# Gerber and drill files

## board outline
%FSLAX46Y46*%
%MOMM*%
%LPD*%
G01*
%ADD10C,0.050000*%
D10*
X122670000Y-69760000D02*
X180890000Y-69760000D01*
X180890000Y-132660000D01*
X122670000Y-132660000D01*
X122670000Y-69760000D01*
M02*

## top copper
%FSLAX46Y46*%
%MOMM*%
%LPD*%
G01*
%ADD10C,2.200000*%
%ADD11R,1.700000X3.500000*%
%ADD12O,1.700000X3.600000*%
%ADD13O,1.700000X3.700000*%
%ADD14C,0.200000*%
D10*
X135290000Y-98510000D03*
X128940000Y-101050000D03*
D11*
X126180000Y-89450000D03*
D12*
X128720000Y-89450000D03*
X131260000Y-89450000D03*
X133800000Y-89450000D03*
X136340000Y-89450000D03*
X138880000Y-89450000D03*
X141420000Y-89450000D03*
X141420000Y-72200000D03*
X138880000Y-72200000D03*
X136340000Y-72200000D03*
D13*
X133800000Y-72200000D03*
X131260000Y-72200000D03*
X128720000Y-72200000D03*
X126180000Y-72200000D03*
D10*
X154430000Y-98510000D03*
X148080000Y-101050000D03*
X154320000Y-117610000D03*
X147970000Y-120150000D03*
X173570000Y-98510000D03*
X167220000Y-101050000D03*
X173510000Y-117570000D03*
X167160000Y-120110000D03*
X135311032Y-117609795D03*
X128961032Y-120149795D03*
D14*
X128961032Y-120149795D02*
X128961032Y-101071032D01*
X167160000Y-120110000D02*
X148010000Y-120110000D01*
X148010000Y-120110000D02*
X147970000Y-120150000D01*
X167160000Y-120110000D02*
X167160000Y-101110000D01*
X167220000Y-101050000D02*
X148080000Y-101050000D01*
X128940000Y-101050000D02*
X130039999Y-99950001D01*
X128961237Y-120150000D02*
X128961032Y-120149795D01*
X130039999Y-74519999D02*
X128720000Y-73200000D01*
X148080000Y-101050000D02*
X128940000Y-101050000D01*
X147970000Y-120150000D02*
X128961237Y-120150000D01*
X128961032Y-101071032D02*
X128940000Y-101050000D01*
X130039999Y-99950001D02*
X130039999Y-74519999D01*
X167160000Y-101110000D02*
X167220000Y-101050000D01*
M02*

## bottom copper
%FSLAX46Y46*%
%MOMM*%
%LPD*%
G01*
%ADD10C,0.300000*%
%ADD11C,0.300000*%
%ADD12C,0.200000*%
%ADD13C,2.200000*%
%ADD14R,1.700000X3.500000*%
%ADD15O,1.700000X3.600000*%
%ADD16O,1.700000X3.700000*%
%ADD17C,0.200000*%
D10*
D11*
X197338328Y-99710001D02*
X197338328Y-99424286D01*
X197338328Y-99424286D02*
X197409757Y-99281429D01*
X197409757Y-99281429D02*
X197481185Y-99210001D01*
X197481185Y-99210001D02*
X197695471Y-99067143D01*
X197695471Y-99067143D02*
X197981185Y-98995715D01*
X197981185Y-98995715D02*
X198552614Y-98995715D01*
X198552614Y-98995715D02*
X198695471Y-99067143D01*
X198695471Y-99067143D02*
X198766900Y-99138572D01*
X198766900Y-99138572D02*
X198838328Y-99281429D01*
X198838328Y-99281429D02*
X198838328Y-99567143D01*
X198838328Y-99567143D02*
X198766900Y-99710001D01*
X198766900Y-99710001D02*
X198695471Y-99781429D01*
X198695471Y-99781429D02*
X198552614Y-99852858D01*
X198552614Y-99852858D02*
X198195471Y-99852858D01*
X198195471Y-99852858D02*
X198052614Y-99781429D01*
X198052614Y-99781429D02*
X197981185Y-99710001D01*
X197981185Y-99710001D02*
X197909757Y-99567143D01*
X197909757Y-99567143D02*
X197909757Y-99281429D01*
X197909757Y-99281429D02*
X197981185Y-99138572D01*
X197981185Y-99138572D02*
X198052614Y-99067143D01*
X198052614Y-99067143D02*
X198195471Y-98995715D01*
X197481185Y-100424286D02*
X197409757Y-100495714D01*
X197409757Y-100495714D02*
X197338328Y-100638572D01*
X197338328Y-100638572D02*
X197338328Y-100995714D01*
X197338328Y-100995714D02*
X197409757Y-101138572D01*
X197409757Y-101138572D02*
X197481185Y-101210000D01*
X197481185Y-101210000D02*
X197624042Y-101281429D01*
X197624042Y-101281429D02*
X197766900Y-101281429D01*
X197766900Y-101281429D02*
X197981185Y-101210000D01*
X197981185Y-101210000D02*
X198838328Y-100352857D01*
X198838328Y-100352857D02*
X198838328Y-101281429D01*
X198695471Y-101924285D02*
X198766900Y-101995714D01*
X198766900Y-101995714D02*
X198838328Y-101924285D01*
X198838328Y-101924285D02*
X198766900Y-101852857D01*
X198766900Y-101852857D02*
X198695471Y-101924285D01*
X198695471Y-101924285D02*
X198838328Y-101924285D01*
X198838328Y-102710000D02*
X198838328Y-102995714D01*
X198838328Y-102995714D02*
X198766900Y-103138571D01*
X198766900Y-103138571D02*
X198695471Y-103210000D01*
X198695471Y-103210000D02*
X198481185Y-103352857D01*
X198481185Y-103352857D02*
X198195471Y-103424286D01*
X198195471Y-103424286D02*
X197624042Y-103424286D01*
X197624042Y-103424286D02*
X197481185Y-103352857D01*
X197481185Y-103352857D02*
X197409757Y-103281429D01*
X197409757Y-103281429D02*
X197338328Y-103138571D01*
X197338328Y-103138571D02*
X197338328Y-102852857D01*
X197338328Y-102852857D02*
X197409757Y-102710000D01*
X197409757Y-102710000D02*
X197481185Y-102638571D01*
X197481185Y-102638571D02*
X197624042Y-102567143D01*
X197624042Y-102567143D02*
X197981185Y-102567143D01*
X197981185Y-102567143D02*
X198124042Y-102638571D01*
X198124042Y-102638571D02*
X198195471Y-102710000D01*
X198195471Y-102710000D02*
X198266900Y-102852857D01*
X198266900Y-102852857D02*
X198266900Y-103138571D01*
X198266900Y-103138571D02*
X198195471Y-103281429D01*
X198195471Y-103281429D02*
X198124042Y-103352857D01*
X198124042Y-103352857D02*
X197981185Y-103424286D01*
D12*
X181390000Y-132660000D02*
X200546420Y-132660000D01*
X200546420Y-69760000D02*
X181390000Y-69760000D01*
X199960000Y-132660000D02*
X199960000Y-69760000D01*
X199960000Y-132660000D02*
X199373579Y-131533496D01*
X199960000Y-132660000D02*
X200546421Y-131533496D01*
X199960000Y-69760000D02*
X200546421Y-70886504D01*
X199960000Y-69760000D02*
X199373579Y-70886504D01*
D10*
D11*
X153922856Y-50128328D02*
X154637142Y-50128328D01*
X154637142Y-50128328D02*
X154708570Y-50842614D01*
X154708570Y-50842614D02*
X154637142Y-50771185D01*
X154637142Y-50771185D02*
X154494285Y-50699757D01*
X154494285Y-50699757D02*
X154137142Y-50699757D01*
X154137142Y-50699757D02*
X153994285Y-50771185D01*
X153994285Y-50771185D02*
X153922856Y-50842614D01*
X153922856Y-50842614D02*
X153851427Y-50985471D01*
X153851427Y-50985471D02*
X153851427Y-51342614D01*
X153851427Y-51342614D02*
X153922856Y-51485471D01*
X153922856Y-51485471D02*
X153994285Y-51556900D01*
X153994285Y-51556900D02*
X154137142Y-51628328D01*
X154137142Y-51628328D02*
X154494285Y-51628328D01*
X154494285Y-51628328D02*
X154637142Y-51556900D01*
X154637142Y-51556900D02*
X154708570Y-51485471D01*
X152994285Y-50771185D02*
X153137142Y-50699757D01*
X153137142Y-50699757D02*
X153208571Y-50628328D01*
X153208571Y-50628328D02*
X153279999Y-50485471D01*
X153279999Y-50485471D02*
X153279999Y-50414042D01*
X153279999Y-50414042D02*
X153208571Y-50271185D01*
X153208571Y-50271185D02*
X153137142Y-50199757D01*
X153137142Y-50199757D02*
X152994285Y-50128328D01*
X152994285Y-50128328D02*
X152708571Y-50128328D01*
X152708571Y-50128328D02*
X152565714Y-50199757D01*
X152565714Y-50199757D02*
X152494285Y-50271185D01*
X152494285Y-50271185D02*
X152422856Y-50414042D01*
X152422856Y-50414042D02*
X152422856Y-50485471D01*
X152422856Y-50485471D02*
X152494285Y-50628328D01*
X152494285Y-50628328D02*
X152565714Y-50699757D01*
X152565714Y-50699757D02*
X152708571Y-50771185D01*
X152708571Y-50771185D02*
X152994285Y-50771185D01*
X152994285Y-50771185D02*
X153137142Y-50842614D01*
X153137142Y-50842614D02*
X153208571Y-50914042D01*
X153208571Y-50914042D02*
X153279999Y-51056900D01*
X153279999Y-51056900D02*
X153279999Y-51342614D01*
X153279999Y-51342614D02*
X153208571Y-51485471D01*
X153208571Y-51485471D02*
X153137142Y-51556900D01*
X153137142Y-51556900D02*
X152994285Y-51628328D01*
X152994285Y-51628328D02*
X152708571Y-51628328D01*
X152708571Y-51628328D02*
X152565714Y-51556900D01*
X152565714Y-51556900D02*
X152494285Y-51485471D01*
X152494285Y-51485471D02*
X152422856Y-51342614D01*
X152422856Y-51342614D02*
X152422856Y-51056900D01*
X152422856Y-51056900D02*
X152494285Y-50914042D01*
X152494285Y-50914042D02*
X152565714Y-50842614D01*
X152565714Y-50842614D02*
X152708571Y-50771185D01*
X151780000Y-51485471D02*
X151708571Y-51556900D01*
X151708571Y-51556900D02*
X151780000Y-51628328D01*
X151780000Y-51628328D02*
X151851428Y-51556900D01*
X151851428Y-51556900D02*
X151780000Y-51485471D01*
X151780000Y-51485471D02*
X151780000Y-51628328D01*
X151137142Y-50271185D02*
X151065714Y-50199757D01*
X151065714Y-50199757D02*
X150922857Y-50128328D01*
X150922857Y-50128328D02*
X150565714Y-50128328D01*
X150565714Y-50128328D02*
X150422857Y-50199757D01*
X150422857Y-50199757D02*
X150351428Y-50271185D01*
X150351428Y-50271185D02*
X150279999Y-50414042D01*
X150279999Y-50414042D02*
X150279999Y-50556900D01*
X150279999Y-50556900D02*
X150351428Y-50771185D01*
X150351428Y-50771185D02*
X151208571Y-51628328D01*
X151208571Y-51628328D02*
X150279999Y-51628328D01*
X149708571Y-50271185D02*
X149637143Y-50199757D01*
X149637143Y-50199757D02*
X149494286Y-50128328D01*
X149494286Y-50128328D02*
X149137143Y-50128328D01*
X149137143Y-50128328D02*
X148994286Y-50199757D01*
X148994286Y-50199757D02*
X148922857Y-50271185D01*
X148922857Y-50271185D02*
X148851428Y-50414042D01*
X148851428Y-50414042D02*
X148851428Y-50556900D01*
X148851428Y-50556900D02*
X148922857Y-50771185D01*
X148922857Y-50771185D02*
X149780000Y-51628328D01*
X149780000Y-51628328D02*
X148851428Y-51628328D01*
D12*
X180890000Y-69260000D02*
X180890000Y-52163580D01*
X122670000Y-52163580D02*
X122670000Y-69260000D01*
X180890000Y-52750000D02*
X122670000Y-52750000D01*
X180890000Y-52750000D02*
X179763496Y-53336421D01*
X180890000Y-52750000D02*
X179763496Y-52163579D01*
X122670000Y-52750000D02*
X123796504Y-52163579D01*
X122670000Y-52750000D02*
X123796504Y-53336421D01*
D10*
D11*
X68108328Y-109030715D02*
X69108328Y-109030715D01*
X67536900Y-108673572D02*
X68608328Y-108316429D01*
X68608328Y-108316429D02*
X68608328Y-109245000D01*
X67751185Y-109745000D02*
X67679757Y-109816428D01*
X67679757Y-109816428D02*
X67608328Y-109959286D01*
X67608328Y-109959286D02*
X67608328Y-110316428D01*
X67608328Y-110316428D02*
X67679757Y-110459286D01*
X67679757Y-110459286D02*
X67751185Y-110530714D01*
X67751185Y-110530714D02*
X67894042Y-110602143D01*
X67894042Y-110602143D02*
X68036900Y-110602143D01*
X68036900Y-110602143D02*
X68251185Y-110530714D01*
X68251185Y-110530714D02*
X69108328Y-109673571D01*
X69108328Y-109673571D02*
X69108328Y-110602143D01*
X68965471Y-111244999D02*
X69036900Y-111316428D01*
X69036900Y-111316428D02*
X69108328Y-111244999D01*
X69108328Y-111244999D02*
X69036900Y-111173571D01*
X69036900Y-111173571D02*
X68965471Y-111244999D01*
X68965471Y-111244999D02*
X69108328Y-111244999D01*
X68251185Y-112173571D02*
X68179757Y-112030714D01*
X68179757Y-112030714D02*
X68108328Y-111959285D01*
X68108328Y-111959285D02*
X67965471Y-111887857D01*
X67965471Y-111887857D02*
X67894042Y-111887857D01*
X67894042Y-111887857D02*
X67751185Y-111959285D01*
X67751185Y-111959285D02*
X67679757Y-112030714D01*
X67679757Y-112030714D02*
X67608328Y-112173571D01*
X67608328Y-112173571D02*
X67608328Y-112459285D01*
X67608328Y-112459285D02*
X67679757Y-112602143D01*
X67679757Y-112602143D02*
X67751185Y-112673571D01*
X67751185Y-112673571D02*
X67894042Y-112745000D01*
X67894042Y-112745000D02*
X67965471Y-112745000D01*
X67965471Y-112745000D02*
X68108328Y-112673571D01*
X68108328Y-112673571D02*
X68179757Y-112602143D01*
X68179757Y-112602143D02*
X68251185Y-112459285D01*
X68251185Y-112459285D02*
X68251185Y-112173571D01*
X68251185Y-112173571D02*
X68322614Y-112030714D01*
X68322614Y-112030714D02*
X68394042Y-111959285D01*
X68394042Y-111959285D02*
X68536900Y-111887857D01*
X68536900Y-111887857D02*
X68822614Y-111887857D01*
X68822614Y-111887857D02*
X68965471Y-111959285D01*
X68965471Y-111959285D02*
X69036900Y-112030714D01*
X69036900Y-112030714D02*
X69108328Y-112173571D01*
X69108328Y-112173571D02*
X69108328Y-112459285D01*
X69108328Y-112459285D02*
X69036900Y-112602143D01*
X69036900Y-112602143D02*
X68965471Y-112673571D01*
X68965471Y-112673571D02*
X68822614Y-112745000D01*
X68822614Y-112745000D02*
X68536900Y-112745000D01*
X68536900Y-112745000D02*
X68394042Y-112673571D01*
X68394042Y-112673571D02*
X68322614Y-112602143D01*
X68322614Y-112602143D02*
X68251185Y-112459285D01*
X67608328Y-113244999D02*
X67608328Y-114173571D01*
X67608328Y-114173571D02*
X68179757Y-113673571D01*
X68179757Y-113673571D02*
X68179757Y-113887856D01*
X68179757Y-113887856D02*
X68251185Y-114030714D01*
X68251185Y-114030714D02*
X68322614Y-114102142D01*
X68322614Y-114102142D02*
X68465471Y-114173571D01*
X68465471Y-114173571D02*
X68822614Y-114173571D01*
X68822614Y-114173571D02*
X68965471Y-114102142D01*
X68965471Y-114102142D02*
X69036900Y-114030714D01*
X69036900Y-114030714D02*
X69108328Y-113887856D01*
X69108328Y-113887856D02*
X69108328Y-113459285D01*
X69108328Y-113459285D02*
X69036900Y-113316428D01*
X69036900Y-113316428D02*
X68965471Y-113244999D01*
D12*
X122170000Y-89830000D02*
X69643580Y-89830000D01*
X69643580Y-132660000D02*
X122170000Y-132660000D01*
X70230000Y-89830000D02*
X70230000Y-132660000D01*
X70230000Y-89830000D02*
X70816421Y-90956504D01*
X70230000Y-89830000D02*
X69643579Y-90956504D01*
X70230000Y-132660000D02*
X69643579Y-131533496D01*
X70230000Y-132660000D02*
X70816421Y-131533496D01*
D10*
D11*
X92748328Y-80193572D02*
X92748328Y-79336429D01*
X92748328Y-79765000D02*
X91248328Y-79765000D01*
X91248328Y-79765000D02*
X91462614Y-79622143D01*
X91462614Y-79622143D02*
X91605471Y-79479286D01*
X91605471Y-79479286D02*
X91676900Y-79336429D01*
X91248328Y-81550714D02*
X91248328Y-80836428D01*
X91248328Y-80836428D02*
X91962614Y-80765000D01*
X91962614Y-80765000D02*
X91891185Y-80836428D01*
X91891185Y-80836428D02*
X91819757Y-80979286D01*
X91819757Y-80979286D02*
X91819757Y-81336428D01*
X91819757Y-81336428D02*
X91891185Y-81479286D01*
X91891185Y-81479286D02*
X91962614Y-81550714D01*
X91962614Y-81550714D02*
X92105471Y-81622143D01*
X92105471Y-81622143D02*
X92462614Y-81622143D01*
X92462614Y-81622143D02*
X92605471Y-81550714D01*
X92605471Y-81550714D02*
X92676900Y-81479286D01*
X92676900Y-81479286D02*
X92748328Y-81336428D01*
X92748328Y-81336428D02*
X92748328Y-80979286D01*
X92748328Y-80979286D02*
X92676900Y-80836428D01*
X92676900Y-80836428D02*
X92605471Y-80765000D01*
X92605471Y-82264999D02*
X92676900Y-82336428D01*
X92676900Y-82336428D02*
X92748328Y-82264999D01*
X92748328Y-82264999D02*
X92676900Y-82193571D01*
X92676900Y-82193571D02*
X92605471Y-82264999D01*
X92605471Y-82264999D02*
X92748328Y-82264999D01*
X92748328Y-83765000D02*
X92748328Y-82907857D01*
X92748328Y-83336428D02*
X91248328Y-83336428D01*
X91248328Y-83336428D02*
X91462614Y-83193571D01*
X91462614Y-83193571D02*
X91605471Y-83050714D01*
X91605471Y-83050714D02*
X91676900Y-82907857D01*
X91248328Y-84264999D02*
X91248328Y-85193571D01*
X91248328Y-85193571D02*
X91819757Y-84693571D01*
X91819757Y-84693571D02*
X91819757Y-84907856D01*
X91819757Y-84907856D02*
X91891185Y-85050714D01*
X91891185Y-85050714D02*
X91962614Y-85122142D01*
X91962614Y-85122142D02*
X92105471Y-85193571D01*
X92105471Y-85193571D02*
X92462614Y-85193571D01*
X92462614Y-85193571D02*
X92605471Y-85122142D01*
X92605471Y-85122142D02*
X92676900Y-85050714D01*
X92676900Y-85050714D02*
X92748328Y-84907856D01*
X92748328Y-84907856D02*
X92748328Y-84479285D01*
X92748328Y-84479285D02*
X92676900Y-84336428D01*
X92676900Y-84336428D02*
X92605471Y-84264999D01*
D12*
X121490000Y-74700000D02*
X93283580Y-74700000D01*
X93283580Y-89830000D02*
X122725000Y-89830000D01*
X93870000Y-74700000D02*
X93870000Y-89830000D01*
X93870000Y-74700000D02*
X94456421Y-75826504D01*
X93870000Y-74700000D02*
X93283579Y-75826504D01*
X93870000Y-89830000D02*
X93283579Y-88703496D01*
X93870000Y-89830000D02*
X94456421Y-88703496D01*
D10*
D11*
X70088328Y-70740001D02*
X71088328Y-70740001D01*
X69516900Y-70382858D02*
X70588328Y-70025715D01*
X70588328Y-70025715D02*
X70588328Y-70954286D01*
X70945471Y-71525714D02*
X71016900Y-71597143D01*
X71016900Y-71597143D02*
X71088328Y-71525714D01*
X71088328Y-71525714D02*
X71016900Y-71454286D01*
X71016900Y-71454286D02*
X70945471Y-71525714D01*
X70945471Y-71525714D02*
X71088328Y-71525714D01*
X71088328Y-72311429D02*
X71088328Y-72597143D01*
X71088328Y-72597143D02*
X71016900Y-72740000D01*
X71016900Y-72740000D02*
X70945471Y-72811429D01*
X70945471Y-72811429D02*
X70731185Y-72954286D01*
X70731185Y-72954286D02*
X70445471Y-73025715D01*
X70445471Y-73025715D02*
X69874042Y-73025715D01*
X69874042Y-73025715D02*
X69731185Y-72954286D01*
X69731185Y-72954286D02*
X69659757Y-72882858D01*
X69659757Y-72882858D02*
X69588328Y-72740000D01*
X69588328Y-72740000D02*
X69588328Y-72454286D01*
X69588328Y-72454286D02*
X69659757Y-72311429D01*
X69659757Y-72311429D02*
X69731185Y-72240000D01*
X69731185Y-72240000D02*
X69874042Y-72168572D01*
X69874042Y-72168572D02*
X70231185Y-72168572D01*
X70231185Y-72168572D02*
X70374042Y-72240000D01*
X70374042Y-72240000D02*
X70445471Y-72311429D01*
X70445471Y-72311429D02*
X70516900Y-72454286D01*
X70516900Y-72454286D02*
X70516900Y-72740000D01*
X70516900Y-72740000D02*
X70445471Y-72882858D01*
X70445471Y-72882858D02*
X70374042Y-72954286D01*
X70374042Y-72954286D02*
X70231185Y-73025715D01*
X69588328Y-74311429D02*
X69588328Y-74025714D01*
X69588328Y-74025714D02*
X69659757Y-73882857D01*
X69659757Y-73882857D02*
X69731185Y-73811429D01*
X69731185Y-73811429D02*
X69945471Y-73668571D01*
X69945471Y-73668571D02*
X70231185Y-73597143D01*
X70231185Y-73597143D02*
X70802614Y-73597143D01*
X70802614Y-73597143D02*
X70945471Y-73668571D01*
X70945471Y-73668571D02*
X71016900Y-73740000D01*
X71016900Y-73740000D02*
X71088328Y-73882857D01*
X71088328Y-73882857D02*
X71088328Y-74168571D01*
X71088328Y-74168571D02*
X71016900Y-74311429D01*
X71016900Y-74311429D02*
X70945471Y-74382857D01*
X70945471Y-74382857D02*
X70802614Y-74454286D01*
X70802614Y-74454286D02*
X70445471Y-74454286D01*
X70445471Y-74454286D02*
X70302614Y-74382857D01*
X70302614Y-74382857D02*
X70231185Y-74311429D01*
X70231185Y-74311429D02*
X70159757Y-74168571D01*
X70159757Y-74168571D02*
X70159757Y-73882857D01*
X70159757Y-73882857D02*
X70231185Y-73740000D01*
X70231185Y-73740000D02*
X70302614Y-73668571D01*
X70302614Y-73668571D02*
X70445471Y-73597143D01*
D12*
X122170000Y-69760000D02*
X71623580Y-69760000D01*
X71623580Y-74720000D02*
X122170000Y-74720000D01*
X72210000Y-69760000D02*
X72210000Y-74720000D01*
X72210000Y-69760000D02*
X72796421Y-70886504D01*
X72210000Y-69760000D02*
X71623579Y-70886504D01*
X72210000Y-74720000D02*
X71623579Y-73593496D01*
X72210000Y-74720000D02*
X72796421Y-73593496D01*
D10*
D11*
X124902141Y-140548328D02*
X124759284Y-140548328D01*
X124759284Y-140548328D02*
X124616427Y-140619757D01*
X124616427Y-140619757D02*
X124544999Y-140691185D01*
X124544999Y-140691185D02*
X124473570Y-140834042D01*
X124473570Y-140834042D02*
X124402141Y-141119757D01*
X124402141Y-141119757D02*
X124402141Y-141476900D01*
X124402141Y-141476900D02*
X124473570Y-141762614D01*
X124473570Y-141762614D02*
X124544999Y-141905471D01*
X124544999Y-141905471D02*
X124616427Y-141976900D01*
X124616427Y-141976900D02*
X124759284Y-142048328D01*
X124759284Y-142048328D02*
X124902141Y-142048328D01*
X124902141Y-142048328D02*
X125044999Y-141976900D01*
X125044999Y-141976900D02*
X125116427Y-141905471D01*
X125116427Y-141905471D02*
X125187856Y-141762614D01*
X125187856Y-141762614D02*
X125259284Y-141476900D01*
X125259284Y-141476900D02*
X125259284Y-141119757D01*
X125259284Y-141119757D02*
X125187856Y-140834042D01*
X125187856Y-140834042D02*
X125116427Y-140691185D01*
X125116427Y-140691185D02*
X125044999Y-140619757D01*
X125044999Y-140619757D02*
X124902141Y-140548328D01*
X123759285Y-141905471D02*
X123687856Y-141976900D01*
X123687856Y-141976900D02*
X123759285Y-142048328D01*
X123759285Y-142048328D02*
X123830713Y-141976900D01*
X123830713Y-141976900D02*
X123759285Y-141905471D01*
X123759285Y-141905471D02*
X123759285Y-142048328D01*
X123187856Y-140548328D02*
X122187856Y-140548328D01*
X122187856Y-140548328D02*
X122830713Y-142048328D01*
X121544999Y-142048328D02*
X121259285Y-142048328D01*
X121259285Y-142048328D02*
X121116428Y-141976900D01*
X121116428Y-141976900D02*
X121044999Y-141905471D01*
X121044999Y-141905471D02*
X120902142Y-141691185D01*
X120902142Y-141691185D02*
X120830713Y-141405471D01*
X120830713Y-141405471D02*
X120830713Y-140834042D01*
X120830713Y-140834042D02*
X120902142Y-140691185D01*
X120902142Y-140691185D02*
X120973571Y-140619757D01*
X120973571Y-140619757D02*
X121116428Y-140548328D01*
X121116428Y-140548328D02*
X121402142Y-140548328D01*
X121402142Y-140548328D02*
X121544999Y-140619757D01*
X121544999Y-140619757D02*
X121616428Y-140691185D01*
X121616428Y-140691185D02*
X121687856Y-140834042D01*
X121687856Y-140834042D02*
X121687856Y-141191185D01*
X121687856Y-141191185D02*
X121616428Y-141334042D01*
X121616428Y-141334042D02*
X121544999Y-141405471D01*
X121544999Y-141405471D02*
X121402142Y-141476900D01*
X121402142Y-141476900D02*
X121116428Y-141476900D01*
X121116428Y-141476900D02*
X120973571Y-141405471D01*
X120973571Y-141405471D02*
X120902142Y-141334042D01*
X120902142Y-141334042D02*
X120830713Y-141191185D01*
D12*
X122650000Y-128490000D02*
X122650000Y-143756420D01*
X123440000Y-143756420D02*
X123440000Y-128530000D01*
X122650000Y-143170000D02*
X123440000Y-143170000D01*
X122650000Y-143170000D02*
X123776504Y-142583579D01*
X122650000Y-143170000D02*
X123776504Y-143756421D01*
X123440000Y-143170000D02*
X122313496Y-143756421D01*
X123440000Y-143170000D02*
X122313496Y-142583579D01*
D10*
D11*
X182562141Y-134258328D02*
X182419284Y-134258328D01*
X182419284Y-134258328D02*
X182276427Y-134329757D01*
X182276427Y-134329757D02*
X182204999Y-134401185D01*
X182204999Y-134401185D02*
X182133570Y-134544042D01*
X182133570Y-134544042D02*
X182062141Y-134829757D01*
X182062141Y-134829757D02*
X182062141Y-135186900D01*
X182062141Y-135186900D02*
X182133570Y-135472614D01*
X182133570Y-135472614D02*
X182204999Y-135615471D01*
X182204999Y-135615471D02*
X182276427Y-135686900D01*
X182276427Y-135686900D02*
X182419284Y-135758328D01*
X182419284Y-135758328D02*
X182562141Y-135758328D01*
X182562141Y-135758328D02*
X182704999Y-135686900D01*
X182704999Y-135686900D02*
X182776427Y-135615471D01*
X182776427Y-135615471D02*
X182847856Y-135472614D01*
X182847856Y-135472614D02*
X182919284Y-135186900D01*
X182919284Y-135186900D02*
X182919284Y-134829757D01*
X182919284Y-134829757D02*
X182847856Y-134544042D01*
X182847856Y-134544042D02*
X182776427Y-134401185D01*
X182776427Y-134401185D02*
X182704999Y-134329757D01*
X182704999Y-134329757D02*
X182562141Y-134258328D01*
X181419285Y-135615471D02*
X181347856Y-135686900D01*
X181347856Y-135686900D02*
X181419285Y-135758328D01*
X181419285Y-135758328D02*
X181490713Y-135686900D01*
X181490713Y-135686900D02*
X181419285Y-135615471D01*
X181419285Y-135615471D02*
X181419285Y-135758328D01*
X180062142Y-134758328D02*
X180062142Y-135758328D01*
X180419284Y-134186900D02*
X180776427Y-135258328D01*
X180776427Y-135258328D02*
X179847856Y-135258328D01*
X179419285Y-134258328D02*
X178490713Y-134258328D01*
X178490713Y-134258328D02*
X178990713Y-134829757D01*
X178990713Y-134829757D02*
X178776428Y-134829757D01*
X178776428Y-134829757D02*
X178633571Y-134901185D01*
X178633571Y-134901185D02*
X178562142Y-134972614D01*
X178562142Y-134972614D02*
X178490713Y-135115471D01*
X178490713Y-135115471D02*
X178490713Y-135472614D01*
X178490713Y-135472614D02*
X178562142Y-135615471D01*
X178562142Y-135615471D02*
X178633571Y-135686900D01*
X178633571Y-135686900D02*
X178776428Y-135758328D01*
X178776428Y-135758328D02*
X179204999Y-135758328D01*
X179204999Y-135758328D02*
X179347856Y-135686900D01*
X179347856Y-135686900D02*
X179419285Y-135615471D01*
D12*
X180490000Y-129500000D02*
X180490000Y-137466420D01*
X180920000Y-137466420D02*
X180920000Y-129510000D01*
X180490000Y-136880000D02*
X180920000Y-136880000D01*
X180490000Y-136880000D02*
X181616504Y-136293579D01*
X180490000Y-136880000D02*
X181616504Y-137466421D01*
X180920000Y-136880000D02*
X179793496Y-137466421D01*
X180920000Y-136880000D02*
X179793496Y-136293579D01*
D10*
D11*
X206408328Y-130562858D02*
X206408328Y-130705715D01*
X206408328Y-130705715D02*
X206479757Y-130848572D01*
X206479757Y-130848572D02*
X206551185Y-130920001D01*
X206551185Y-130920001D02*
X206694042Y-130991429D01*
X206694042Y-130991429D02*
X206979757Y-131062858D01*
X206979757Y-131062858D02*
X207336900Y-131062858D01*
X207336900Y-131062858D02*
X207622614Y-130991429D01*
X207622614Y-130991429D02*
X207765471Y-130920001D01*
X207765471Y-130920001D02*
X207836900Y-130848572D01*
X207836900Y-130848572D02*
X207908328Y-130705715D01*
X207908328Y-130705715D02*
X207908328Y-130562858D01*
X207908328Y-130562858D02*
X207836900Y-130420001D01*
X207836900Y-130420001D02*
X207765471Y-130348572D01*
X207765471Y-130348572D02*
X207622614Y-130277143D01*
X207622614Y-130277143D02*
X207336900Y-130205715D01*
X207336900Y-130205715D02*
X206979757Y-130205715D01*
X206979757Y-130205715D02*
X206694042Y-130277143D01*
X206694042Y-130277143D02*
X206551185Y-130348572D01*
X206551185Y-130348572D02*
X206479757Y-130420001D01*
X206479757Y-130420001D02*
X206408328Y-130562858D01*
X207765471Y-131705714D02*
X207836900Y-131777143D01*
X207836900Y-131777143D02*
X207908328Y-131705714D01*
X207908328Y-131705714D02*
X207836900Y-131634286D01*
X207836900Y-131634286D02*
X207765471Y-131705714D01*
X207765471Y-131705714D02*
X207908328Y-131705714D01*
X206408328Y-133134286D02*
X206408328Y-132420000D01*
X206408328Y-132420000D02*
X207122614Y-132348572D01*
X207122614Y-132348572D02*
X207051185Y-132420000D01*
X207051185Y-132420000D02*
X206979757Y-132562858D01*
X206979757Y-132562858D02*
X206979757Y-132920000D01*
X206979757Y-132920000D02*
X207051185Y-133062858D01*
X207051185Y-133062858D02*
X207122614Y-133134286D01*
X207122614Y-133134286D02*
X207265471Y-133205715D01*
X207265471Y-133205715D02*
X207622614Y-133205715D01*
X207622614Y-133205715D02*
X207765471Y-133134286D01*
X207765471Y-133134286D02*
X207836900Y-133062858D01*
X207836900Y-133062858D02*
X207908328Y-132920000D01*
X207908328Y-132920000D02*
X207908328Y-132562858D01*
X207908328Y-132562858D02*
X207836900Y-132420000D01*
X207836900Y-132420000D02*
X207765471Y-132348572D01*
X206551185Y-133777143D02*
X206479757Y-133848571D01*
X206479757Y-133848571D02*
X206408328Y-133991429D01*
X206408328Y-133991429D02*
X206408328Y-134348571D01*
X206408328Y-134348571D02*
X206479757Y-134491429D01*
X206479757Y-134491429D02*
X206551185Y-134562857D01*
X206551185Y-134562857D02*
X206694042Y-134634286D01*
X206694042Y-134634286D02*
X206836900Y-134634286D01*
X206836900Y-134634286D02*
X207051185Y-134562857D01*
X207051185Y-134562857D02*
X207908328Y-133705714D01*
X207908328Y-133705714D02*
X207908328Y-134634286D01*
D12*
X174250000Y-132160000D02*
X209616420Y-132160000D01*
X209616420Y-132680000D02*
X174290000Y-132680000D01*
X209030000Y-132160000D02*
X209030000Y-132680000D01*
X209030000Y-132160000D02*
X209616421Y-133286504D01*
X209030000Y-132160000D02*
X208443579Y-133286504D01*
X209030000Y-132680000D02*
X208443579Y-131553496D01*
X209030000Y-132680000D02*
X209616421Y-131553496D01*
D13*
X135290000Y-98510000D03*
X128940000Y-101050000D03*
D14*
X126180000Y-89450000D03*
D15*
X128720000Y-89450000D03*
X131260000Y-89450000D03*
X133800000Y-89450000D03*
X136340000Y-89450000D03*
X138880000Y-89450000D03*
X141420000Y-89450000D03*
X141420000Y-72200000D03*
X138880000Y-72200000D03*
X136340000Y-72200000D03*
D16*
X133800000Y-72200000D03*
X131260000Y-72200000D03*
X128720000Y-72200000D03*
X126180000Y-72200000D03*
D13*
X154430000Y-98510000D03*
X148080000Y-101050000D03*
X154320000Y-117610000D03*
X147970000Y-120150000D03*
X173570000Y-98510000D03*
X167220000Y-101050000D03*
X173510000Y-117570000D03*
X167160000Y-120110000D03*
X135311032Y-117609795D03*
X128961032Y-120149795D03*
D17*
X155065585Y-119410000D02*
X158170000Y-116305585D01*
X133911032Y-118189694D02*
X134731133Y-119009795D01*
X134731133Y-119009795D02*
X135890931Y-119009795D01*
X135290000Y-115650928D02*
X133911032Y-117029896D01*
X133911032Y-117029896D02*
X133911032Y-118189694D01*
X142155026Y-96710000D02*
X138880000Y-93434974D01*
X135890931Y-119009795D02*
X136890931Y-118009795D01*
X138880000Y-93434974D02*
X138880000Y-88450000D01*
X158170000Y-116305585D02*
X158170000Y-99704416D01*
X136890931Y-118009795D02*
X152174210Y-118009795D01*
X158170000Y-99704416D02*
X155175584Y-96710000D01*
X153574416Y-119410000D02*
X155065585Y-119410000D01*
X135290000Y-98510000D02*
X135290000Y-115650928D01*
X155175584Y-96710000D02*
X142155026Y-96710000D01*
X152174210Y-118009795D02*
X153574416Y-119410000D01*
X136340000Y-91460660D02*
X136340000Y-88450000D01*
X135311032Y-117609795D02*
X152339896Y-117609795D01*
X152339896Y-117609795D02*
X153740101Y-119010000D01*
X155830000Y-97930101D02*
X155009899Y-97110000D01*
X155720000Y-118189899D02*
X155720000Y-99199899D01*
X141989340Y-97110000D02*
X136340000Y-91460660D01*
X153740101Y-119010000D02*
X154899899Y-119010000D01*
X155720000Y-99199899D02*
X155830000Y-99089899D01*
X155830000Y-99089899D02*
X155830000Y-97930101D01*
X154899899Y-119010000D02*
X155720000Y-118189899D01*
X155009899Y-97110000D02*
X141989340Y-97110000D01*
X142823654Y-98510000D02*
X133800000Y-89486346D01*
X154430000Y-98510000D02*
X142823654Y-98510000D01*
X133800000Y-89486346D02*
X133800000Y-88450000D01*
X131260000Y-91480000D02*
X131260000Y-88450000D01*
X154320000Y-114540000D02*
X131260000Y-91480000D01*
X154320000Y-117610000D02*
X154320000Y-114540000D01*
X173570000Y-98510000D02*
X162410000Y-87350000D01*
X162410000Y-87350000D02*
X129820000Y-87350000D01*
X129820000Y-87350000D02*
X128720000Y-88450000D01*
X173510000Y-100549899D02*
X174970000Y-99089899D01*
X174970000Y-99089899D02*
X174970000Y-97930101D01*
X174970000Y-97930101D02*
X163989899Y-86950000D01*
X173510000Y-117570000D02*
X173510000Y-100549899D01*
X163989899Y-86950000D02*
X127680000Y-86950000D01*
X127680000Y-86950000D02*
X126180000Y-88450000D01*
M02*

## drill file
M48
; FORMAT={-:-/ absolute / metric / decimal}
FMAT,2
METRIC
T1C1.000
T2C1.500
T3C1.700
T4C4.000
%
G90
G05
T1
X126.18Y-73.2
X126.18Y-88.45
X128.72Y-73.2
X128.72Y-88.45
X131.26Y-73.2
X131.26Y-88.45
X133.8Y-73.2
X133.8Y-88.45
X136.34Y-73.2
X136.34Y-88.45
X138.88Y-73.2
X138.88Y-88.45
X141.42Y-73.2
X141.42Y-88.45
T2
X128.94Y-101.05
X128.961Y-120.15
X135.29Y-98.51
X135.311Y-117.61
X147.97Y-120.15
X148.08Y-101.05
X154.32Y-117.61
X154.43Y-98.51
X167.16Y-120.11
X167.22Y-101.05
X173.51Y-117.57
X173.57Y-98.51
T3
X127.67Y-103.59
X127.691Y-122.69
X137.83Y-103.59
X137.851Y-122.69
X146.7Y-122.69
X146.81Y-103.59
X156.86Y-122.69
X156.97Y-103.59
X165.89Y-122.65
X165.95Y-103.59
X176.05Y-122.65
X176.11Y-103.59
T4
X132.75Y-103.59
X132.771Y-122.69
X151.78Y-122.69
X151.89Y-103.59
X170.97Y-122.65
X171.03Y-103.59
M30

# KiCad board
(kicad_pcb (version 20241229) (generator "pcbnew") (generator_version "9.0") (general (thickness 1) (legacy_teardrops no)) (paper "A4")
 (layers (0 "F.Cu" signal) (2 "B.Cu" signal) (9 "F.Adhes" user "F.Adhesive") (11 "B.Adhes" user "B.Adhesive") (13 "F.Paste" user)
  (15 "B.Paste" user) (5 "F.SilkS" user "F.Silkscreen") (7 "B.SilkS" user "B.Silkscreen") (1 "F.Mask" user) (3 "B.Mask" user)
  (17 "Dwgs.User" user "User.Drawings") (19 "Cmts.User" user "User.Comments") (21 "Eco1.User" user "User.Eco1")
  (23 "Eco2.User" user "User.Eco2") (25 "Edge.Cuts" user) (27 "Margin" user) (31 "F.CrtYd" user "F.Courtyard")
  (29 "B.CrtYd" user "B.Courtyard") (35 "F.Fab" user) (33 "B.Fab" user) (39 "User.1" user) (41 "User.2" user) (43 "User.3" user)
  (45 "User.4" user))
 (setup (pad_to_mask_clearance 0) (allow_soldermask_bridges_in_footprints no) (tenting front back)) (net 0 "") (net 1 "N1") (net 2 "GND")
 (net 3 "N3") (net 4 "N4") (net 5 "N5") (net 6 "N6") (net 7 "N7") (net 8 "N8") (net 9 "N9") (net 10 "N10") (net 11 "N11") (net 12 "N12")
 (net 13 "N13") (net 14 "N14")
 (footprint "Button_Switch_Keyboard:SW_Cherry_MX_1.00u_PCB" (layer "F.Cu") (at 135.29 98.51)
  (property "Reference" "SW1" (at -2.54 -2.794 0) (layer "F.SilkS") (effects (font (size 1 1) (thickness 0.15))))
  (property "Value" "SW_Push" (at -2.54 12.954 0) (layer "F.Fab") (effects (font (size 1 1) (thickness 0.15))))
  (pad "" np_thru_hole circle (at -7.62 5.08) (size 1.7 1.7) (drill 1.7) (layers "*.Cu" "*.Mask"))
  (pad "" np_thru_hole circle (at -2.54 5.08) (size 4 4) (drill 4) (layers "*.Cu" "*.Mask"))
  (pad "" np_thru_hole circle (at 2.54 5.08) (size 1.7 1.7) (drill 1.7) (layers "*.Cu" "*.Mask"))
  (pad "1" thru_hole circle (at 0 0) (size 2.2 2.2) (drill 1.5) (layers "*.Cu" "*.Mask") (remove_unused_layers no) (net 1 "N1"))
  (pad "2" thru_hole circle (at -6.35 2.54) (size 2.2 2.2) (drill 1.5) (layers "*.Cu" "*.Mask") (remove_unused_layers no) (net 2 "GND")))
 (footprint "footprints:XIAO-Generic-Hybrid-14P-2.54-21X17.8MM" (layer "F.Cu") (at 133.8 80.825 90)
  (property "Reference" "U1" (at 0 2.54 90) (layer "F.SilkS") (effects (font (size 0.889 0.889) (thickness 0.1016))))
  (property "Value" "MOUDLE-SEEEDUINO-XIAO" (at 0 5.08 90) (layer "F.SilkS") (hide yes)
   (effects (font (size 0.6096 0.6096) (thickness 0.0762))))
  (pad "1" thru_hole rect (at -7.625 -7.62 90) (size 3.5 1.7) (drill 1 (offset -1 0)) (layers "*.Cu" "*.Mask") (remove_unused_layers no)
   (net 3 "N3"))
  (pad "2" thru_hole oval (at -7.625 -5.08 90) (size 3.6 1.7) (drill 1 (offset -1 0)) (layers "*.Cu" "*.Mask") (remove_unused_layers no)
   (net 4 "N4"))
  (pad "3" thru_hole oval (at -7.625 -2.54 90) (size 3.6 1.7) (drill 1 (offset -1 0)) (layers "*.Cu" "*.Mask") (remove_unused_layers no)
   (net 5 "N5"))
  (pad "4" thru_hole oval (at -7.625 0 90) (size 3.6 1.7) (drill 1 (offset -1 0)) (layers "*.Cu" "*.Mask") (remove_unused_layers no)
   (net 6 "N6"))
  (pad "5" thru_hole oval (at -7.625 2.54 90) (size 3.6 1.7) (drill 1 (offset -1 0)) (layers "*.Cu" "*.Mask") (remove_unused_layers no)
   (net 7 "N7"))
  (pad "6" thru_hole oval (at -7.625 5.08 270) (size 3.6 1.7) (drill 1 (offset 1 0)) (layers "*.Cu" "*.Mask") (remove_unused_layers no)
   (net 1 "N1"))
  (pad "7" thru_hole oval (at -7.625 7.62 90) (size 3.6 1.7) (drill 1 (offset -1 0)) (layers "*.Cu" "*.Mask") (remove_unused_layers no)
   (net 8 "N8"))
  (pad "8" thru_hole oval (at 7.625 7.62 90) (size 3.6 1.7) (drill 1 (offset 1 0)) (layers "*.Cu" "*.Mask") (remove_unused_layers no)
   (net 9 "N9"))
  (pad "9" thru_hole oval (at 7.625 5.08 90) (size 3.6 1.7) (drill 1 (offset 1 0)) (layers "*.Cu" "*.Mask") (remove_unused_layers no)
   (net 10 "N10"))
  (pad "10" thru_hole oval (at 7.625 2.54 90) (size 3.6 1.7) (drill 1 (offset 1 0)) (layers "*.Cu" "*.Mask") (remove_unused_layers no)
   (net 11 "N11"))
  (pad "11" thru_hole oval (at 7.625 0 90) (size 3.7 1.7) (drill 1 (offset 1 0)) (layers "*.Cu" "*.Mask") (remove_unused_layers no)
   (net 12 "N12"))
  (pad "12" thru_hole oval (at 7.625 -2.54 90) (size 3.7 1.7) (drill 1 (offset 1 0)) (layers "*.Cu" "*.Mask") (remove_unused_layers no)
   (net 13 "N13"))
  (pad "13" thru_hole oval (at 7.625 -5.08 90) (size 3.7 1.7) (drill 1 (offset 1 0)) (layers "*.Cu" "*.Mask") (remove_unused_layers no)
   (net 2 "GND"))
  (pad "14" thru_hole oval (at 7.625 -7.62 90) (size 3.7 1.7) (drill 1 (offset 1 0)) (layers "*.Cu" "*.Mask") (remove_unused_layers no)
   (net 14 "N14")))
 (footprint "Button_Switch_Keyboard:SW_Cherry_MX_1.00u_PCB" (layer "F.Cu") (at 154.43 98.51)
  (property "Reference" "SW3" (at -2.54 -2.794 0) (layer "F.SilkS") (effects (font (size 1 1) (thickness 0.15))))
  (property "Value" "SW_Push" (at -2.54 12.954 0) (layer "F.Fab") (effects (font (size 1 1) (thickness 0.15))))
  (pad "" np_thru_hole circle (at -7.62 5.08) (size 1.7 1.7) (drill 1.7) (layers "*.Cu" "*.Mask"))
  (pad "" np_thru_hole circle (at -2.54 5.08) (size 4 4) (drill 4) (layers "*.Cu" "*.Mask"))
  (pad "" np_thru_hole circle (at 2.54 5.08) (size 1.7 1.7) (drill 1.7) (layers "*.Cu" "*.Mask"))
  (pad "1" thru_hole circle (at 0 0) (size 2.2 2.2) (drill 1.5) (layers "*.Cu" "*.Mask") (remove_unused_layers no) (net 6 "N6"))
  (pad "2" thru_hole circle (at -6.35 2.54) (size 2.2 2.2) (drill 1.5) (layers "*.Cu" "*.Mask") (remove_unused_layers no) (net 2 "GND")))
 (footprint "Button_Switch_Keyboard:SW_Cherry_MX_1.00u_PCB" (layer "F.Cu") (at 154.32 117.61)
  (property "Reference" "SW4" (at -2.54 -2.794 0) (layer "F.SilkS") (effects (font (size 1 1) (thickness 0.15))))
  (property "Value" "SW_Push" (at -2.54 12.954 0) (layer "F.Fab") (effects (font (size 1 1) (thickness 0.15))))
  (pad "" np_thru_hole circle (at -7.62 5.08) (size 1.7 1.7) (drill 1.7) (layers "*.Cu" "*.Mask"))
  (pad "" np_thru_hole circle (at -2.54 5.08) (size 4 4) (drill 4) (layers "*.Cu" "*.Mask"))
  (pad "" np_thru_hole circle (at 2.54 5.08) (size 1.7 1.7) (drill 1.7) (layers "*.Cu" "*.Mask"))
  (pad "1" thru_hole circle (at 0 0) (size 2.2 2.2) (drill 1.5) (layers "*.Cu" "*.Mask") (remove_unused_layers no) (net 5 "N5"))
  (pad "2" thru_hole circle (at -6.35 2.54) (size 2.2 2.2) (drill 1.5) (layers "*.Cu" "*.Mask") (remove_unused_layers no) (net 2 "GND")))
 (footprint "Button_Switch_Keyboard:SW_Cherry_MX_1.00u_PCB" (layer "F.Cu") (at 173.57 98.51)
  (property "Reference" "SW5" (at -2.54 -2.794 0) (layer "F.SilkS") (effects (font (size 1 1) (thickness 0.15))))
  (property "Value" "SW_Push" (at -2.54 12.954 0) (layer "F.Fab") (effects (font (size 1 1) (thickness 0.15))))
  (pad "" np_thru_hole circle (at -7.62 5.08) (size 1.7 1.7) (drill 1.7) (layers "*.Cu" "*.Mask"))
  (pad "" np_thru_hole circle (at -2.54 5.08) (size 4 4) (drill 4) (layers "*.Cu" "*.Mask"))
  (pad "" np_thru_hole circle (at 2.54 5.08) (size 1.7 1.7) (drill 1.7) (layers "*.Cu" "*.Mask"))
  (pad "1" thru_hole circle (at 0 0) (size 2.2 2.2) (drill 1.5) (layers "*.Cu" "*.Mask") (remove_unused_layers no) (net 4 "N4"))
  (pad "2" thru_hole circle (at -6.35 2.54) (size 2.2 2.2) (drill 1.5) (layers "*.Cu" "*.Mask") (remove_unused_layers no) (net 2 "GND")))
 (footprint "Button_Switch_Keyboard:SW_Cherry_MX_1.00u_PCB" (layer "F.Cu") (at 173.51 117.57)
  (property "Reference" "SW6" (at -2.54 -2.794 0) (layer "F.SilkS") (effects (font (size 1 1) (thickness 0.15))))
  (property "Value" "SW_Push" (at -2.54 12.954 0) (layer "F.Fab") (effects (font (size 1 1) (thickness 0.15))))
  (pad "" np_thru_hole circle (at -7.62 5.08) (size 1.7 1.7) (drill 1.7) (layers "*.Cu" "*.Mask"))
  (pad "" np_thru_hole circle (at -2.54 5.08) (size 4 4) (drill 4) (layers "*.Cu" "*.Mask"))
  (pad "" np_thru_hole circle (at 2.54 5.08) (size 1.7 1.7) (drill 1.7) (layers "*.Cu" "*.Mask"))
  (pad "1" thru_hole circle (at 0 0) (size 2.2 2.2) (drill 1.5) (layers "*.Cu" "*.Mask") (remove_unused_layers no) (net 3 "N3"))
  (pad "2" thru_hole circle (at -6.35 2.54) (size 2.2 2.2) (drill 1.5) (layers "*.Cu" "*.Mask") (remove_unused_layers no) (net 2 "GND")))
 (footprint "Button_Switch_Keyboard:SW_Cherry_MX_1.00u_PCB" (layer "F.Cu") (at 135.311032 117.609795)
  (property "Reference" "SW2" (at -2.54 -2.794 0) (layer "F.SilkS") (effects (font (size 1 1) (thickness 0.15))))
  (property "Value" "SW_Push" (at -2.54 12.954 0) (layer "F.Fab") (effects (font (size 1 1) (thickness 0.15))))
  (pad "" np_thru_hole circle (at -7.62 5.08) (size 1.7 1.7) (drill 1.7) (layers "*.Cu" "*.Mask"))
  (pad "" np_thru_hole circle (at -2.54 5.08) (size 4 4) (drill 4) (layers "*.Cu" "*.Mask"))
  (pad "" np_thru_hole circle (at 2.54 5.08) (size 1.7 1.7) (drill 1.7) (layers "*.Cu" "*.Mask"))
  (pad "1" thru_hole circle (at 0 0) (size 2.2 2.2) (drill 1.5) (layers "*.Cu" "*.Mask") (remove_unused_layers no) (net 7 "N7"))
  (pad "2" thru_hole circle (at -6.35 2.54) (size 2.2 2.2) (drill 1.5) (layers "*.Cu" "*.Mask") (remove_unused_layers no) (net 2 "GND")))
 (gr_rect (start 122.67 69.76) (end 180.89 132.66) (stroke (width 0.05) (type default)) (fill no) (layer "Edge.Cuts"))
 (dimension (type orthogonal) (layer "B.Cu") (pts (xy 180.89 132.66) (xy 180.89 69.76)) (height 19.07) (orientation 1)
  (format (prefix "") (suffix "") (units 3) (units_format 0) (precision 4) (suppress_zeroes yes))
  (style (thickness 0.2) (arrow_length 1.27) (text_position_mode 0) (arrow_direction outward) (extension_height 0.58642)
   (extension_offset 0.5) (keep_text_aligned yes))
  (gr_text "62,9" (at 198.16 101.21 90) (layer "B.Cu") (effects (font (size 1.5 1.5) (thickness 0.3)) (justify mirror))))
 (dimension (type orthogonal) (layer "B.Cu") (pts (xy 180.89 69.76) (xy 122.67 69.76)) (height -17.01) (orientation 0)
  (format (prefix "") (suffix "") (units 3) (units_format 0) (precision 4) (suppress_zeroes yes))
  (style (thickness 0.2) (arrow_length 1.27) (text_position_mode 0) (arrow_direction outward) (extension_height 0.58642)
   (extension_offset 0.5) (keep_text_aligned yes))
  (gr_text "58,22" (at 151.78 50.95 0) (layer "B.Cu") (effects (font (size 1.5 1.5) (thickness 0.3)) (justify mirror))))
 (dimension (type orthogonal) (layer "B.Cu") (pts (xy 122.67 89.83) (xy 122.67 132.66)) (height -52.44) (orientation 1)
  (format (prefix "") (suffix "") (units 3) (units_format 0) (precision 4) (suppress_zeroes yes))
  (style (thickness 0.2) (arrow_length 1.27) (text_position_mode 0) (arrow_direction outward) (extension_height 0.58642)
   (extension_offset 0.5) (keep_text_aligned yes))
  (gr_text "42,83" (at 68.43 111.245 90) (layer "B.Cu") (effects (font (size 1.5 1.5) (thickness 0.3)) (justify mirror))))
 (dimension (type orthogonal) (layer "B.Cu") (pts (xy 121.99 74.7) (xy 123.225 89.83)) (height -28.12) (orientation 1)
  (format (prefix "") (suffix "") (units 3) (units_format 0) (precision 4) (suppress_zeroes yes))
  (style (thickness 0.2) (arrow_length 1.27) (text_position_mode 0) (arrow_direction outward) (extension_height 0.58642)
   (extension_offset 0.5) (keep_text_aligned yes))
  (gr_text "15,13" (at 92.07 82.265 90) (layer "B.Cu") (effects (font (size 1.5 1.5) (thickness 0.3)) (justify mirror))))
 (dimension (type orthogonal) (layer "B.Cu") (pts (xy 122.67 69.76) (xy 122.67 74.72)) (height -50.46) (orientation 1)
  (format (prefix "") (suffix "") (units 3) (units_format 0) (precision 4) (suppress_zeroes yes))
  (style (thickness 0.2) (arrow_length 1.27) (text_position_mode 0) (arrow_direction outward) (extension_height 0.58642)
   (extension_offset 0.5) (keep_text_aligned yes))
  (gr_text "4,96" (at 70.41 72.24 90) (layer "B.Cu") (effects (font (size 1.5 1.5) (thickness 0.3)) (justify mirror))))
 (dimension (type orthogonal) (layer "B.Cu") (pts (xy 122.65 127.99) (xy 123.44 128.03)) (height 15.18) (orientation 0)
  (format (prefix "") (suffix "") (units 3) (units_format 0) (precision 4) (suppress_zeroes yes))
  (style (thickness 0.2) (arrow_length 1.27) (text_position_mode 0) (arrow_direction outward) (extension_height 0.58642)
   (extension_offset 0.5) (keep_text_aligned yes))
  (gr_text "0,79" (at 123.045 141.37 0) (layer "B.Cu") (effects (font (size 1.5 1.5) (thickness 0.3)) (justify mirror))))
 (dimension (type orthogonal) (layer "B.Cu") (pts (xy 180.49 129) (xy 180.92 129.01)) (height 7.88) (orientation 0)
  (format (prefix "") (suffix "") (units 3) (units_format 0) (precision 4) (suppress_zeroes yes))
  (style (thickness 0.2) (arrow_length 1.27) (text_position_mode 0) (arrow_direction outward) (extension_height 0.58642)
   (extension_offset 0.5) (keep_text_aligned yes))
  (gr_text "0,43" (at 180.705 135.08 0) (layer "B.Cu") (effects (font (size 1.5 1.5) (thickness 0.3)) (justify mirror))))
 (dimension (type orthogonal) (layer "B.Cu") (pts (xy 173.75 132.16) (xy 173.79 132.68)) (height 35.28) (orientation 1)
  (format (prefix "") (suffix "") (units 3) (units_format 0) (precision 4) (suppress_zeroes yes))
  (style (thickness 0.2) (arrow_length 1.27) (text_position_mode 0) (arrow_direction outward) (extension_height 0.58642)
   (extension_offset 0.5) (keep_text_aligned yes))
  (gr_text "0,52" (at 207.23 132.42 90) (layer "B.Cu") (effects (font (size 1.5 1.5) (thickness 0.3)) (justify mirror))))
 (segment (start 128.961032 120.149795) (end 128.961032 101.071032) (width 0.2) (layer "F.Cu") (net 2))
 (segment (start 167.16 120.11) (end 148.01 120.11) (width 0.2) (layer "F.Cu") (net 2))
 (segment (start 148.01 120.11) (end 147.97 120.15) (width 0.2) (layer "F.Cu") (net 2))
 (segment (start 167.16 120.11) (end 167.16 101.11) (width 0.2) (layer "F.Cu") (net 2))
 (segment (start 167.22 101.05) (end 148.08 101.05) (width 0.2) (layer "F.Cu") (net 2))
 (segment (start 128.94 101.05) (end 130.039999 99.950001) (width 0.2) (layer "F.Cu") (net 2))
 (segment (start 128.961237 120.15) (end 128.961032 120.149795) (width 0.2) (layer "F.Cu") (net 2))
 (segment (start 130.039999 74.519999) (end 128.72 73.2) (width 0.2) (layer "F.Cu") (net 2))
 (segment (start 148.08 101.05) (end 128.94 101.05) (width 0.2) (layer "F.Cu") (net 2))
 (segment (start 147.97 120.15) (end 128.961237 120.15) (width 0.2) (layer "F.Cu") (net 2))
 (segment (start 128.961032 101.071032) (end 128.94 101.05) (width 0.2) (layer "F.Cu") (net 2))
 (segment (start 130.039999 99.950001) (end 130.039999 74.519999) (width 0.2) (layer "F.Cu") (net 2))
 (segment (start 167.16 101.11) (end 167.22 101.05) (width 0.2) (layer "F.Cu") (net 2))
 (segment (start 155.065585 119.41) (end 158.17 116.305585) (width 0.2) (layer "B.Cu") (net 1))
 (segment (start 133.911032 118.189694) (end 134.731133 119.009795) (width 0.2) (layer "B.Cu") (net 1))
 (segment (start 134.731133 119.009795) (end 135.890931 119.009795) (width 0.2) (layer "B.Cu") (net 1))
 (segment (start 135.29 115.650928) (end 133.911032 117.029896) (width 0.2) (layer "B.Cu") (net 1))
 (segment (start 133.911032 117.029896) (end 133.911032 118.189694) (width 0.2) (layer "B.Cu") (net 1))
 (segment (start 142.155026 96.71) (end 138.88 93.434974) (width 0.2) (layer "B.Cu") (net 1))
 (segment (start 135.890931 119.009795) (end 136.890931 118.009795) (width 0.2) (layer "B.Cu") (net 1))
 (segment (start 138.88 93.434974) (end 138.88 88.45) (width 0.2) (layer "B.Cu") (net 1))
 (segment (start 158.17 116.305585) (end 158.17 99.704416) (width 0.2) (layer "B.Cu") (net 1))
 (segment (start 136.890931 118.009795) (end 152.17421 118.009795) (width 0.2) (layer "B.Cu") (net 1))
 (segment (start 158.17 99.704416) (end 155.175584 96.71) (width 0.2) (layer "B.Cu") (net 1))
 (segment (start 153.574416 119.41) (end 155.065585 119.41) (width 0.2) (layer "B.Cu") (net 1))
 (segment (start 135.29 98.51) (end 135.29 115.650928) (width 0.2) (layer "B.Cu") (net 1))
 (segment (start 155.175584 96.71) (end 142.155026 96.71) (width 0.2) (layer "B.Cu") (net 1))
 (segment (start 152.17421 118.009795) (end 153.574416 119.41) (width 0.2) (layer "B.Cu") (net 1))
 (segment (start 136.34 91.46066) (end 136.34 88.45) (width 0.2) (layer "B.Cu") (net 7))
 (segment (start 135.311032 117.609795) (end 152.339896 117.609795) (width 0.2) (layer "B.Cu") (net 7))
 (segment (start 152.339896 117.609795) (end 153.740101 119.01) (width 0.2) (layer "B.Cu") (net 7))
 (segment (start 155.83 97.930101) (end 155.009899 97.11) (width 0.2) (layer "B.Cu") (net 7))
 (segment (start 155.72 118.189899) (end 155.72 99.199899) (width 0.2) (layer "B.Cu") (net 7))
 (segment (start 141.98934 97.11) (end 136.34 91.46066) (width 0.2) (layer "B.Cu") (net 7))
 (segment (start 153.740101 119.01) (end 154.899899 119.01) (width 0.2) (layer "B.Cu") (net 7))
 (segment (start 155.72 99.199899) (end 155.83 99.089899) (width 0.2) (layer "B.Cu") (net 7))
 (segment (start 155.83 99.089899) (end 155.83 97.930101) (width 0.2) (layer "B.Cu") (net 7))
 (segment (start 154.899899 119.01) (end 155.72 118.189899) (width 0.2) (layer "B.Cu") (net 7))
 (segment (start 155.009899 97.11) (end 141.98934 97.11) (width 0.2) (layer "B.Cu") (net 7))
 (segment (start 142.823654 98.51) (end 133.8 89.486346) (width 0.2) (layer "B.Cu") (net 6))
 (segment (start 154.43 98.51) (end 142.823654 98.51) (width 0.2) (layer "B.Cu") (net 6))
 (segment (start 133.8 89.486346) (end 133.8 88.45) (width 0.2) (layer "B.Cu") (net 6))
 (segment (start 131.26 91.48) (end 131.26 88.45) (width 0.2) (layer "B.Cu") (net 5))
 (segment (start 154.32 114.54) (end 131.26 91.48) (width 0.2) (layer "B.Cu") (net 5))
 (segment (start 154.32 117.61) (end 154.32 114.54) (width 0.2) (layer "B.Cu") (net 5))
 (segment (start 173.57 98.51) (end 162.41 87.35) (width 0.2) (layer "B.Cu") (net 4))
 (segment (start 162.41 87.35) (end 129.82 87.35) (width 0.2) (layer "B.Cu") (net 4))
 (segment (start 129.82 87.35) (end 128.72 88.45) (width 0.2) (layer "B.Cu") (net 4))
 (segment (start 173.51 100.549899) (end 174.97 99.089899) (width 0.2) (layer "B.Cu") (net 3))
 (segment (start 174.97 99.089899) (end 174.97 97.930101) (width 0.2) (layer "B.Cu") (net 3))
 (segment (start 174.97 97.930101) (end 163.989899 86.95) (width 0.2) (layer "B.Cu") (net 3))
 (segment (start 173.51 117.57) (end 173.51 100.549899) (width 0.2) (layer "B.Cu") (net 3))
 (segment (start 163.989899 86.95) (end 127.68 86.95) (width 0.2) (layer "B.Cu") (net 3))
 (segment (start 127.68 86.95) (end 126.18 88.45) (width 0.2) (layer "B.Cu") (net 3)))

